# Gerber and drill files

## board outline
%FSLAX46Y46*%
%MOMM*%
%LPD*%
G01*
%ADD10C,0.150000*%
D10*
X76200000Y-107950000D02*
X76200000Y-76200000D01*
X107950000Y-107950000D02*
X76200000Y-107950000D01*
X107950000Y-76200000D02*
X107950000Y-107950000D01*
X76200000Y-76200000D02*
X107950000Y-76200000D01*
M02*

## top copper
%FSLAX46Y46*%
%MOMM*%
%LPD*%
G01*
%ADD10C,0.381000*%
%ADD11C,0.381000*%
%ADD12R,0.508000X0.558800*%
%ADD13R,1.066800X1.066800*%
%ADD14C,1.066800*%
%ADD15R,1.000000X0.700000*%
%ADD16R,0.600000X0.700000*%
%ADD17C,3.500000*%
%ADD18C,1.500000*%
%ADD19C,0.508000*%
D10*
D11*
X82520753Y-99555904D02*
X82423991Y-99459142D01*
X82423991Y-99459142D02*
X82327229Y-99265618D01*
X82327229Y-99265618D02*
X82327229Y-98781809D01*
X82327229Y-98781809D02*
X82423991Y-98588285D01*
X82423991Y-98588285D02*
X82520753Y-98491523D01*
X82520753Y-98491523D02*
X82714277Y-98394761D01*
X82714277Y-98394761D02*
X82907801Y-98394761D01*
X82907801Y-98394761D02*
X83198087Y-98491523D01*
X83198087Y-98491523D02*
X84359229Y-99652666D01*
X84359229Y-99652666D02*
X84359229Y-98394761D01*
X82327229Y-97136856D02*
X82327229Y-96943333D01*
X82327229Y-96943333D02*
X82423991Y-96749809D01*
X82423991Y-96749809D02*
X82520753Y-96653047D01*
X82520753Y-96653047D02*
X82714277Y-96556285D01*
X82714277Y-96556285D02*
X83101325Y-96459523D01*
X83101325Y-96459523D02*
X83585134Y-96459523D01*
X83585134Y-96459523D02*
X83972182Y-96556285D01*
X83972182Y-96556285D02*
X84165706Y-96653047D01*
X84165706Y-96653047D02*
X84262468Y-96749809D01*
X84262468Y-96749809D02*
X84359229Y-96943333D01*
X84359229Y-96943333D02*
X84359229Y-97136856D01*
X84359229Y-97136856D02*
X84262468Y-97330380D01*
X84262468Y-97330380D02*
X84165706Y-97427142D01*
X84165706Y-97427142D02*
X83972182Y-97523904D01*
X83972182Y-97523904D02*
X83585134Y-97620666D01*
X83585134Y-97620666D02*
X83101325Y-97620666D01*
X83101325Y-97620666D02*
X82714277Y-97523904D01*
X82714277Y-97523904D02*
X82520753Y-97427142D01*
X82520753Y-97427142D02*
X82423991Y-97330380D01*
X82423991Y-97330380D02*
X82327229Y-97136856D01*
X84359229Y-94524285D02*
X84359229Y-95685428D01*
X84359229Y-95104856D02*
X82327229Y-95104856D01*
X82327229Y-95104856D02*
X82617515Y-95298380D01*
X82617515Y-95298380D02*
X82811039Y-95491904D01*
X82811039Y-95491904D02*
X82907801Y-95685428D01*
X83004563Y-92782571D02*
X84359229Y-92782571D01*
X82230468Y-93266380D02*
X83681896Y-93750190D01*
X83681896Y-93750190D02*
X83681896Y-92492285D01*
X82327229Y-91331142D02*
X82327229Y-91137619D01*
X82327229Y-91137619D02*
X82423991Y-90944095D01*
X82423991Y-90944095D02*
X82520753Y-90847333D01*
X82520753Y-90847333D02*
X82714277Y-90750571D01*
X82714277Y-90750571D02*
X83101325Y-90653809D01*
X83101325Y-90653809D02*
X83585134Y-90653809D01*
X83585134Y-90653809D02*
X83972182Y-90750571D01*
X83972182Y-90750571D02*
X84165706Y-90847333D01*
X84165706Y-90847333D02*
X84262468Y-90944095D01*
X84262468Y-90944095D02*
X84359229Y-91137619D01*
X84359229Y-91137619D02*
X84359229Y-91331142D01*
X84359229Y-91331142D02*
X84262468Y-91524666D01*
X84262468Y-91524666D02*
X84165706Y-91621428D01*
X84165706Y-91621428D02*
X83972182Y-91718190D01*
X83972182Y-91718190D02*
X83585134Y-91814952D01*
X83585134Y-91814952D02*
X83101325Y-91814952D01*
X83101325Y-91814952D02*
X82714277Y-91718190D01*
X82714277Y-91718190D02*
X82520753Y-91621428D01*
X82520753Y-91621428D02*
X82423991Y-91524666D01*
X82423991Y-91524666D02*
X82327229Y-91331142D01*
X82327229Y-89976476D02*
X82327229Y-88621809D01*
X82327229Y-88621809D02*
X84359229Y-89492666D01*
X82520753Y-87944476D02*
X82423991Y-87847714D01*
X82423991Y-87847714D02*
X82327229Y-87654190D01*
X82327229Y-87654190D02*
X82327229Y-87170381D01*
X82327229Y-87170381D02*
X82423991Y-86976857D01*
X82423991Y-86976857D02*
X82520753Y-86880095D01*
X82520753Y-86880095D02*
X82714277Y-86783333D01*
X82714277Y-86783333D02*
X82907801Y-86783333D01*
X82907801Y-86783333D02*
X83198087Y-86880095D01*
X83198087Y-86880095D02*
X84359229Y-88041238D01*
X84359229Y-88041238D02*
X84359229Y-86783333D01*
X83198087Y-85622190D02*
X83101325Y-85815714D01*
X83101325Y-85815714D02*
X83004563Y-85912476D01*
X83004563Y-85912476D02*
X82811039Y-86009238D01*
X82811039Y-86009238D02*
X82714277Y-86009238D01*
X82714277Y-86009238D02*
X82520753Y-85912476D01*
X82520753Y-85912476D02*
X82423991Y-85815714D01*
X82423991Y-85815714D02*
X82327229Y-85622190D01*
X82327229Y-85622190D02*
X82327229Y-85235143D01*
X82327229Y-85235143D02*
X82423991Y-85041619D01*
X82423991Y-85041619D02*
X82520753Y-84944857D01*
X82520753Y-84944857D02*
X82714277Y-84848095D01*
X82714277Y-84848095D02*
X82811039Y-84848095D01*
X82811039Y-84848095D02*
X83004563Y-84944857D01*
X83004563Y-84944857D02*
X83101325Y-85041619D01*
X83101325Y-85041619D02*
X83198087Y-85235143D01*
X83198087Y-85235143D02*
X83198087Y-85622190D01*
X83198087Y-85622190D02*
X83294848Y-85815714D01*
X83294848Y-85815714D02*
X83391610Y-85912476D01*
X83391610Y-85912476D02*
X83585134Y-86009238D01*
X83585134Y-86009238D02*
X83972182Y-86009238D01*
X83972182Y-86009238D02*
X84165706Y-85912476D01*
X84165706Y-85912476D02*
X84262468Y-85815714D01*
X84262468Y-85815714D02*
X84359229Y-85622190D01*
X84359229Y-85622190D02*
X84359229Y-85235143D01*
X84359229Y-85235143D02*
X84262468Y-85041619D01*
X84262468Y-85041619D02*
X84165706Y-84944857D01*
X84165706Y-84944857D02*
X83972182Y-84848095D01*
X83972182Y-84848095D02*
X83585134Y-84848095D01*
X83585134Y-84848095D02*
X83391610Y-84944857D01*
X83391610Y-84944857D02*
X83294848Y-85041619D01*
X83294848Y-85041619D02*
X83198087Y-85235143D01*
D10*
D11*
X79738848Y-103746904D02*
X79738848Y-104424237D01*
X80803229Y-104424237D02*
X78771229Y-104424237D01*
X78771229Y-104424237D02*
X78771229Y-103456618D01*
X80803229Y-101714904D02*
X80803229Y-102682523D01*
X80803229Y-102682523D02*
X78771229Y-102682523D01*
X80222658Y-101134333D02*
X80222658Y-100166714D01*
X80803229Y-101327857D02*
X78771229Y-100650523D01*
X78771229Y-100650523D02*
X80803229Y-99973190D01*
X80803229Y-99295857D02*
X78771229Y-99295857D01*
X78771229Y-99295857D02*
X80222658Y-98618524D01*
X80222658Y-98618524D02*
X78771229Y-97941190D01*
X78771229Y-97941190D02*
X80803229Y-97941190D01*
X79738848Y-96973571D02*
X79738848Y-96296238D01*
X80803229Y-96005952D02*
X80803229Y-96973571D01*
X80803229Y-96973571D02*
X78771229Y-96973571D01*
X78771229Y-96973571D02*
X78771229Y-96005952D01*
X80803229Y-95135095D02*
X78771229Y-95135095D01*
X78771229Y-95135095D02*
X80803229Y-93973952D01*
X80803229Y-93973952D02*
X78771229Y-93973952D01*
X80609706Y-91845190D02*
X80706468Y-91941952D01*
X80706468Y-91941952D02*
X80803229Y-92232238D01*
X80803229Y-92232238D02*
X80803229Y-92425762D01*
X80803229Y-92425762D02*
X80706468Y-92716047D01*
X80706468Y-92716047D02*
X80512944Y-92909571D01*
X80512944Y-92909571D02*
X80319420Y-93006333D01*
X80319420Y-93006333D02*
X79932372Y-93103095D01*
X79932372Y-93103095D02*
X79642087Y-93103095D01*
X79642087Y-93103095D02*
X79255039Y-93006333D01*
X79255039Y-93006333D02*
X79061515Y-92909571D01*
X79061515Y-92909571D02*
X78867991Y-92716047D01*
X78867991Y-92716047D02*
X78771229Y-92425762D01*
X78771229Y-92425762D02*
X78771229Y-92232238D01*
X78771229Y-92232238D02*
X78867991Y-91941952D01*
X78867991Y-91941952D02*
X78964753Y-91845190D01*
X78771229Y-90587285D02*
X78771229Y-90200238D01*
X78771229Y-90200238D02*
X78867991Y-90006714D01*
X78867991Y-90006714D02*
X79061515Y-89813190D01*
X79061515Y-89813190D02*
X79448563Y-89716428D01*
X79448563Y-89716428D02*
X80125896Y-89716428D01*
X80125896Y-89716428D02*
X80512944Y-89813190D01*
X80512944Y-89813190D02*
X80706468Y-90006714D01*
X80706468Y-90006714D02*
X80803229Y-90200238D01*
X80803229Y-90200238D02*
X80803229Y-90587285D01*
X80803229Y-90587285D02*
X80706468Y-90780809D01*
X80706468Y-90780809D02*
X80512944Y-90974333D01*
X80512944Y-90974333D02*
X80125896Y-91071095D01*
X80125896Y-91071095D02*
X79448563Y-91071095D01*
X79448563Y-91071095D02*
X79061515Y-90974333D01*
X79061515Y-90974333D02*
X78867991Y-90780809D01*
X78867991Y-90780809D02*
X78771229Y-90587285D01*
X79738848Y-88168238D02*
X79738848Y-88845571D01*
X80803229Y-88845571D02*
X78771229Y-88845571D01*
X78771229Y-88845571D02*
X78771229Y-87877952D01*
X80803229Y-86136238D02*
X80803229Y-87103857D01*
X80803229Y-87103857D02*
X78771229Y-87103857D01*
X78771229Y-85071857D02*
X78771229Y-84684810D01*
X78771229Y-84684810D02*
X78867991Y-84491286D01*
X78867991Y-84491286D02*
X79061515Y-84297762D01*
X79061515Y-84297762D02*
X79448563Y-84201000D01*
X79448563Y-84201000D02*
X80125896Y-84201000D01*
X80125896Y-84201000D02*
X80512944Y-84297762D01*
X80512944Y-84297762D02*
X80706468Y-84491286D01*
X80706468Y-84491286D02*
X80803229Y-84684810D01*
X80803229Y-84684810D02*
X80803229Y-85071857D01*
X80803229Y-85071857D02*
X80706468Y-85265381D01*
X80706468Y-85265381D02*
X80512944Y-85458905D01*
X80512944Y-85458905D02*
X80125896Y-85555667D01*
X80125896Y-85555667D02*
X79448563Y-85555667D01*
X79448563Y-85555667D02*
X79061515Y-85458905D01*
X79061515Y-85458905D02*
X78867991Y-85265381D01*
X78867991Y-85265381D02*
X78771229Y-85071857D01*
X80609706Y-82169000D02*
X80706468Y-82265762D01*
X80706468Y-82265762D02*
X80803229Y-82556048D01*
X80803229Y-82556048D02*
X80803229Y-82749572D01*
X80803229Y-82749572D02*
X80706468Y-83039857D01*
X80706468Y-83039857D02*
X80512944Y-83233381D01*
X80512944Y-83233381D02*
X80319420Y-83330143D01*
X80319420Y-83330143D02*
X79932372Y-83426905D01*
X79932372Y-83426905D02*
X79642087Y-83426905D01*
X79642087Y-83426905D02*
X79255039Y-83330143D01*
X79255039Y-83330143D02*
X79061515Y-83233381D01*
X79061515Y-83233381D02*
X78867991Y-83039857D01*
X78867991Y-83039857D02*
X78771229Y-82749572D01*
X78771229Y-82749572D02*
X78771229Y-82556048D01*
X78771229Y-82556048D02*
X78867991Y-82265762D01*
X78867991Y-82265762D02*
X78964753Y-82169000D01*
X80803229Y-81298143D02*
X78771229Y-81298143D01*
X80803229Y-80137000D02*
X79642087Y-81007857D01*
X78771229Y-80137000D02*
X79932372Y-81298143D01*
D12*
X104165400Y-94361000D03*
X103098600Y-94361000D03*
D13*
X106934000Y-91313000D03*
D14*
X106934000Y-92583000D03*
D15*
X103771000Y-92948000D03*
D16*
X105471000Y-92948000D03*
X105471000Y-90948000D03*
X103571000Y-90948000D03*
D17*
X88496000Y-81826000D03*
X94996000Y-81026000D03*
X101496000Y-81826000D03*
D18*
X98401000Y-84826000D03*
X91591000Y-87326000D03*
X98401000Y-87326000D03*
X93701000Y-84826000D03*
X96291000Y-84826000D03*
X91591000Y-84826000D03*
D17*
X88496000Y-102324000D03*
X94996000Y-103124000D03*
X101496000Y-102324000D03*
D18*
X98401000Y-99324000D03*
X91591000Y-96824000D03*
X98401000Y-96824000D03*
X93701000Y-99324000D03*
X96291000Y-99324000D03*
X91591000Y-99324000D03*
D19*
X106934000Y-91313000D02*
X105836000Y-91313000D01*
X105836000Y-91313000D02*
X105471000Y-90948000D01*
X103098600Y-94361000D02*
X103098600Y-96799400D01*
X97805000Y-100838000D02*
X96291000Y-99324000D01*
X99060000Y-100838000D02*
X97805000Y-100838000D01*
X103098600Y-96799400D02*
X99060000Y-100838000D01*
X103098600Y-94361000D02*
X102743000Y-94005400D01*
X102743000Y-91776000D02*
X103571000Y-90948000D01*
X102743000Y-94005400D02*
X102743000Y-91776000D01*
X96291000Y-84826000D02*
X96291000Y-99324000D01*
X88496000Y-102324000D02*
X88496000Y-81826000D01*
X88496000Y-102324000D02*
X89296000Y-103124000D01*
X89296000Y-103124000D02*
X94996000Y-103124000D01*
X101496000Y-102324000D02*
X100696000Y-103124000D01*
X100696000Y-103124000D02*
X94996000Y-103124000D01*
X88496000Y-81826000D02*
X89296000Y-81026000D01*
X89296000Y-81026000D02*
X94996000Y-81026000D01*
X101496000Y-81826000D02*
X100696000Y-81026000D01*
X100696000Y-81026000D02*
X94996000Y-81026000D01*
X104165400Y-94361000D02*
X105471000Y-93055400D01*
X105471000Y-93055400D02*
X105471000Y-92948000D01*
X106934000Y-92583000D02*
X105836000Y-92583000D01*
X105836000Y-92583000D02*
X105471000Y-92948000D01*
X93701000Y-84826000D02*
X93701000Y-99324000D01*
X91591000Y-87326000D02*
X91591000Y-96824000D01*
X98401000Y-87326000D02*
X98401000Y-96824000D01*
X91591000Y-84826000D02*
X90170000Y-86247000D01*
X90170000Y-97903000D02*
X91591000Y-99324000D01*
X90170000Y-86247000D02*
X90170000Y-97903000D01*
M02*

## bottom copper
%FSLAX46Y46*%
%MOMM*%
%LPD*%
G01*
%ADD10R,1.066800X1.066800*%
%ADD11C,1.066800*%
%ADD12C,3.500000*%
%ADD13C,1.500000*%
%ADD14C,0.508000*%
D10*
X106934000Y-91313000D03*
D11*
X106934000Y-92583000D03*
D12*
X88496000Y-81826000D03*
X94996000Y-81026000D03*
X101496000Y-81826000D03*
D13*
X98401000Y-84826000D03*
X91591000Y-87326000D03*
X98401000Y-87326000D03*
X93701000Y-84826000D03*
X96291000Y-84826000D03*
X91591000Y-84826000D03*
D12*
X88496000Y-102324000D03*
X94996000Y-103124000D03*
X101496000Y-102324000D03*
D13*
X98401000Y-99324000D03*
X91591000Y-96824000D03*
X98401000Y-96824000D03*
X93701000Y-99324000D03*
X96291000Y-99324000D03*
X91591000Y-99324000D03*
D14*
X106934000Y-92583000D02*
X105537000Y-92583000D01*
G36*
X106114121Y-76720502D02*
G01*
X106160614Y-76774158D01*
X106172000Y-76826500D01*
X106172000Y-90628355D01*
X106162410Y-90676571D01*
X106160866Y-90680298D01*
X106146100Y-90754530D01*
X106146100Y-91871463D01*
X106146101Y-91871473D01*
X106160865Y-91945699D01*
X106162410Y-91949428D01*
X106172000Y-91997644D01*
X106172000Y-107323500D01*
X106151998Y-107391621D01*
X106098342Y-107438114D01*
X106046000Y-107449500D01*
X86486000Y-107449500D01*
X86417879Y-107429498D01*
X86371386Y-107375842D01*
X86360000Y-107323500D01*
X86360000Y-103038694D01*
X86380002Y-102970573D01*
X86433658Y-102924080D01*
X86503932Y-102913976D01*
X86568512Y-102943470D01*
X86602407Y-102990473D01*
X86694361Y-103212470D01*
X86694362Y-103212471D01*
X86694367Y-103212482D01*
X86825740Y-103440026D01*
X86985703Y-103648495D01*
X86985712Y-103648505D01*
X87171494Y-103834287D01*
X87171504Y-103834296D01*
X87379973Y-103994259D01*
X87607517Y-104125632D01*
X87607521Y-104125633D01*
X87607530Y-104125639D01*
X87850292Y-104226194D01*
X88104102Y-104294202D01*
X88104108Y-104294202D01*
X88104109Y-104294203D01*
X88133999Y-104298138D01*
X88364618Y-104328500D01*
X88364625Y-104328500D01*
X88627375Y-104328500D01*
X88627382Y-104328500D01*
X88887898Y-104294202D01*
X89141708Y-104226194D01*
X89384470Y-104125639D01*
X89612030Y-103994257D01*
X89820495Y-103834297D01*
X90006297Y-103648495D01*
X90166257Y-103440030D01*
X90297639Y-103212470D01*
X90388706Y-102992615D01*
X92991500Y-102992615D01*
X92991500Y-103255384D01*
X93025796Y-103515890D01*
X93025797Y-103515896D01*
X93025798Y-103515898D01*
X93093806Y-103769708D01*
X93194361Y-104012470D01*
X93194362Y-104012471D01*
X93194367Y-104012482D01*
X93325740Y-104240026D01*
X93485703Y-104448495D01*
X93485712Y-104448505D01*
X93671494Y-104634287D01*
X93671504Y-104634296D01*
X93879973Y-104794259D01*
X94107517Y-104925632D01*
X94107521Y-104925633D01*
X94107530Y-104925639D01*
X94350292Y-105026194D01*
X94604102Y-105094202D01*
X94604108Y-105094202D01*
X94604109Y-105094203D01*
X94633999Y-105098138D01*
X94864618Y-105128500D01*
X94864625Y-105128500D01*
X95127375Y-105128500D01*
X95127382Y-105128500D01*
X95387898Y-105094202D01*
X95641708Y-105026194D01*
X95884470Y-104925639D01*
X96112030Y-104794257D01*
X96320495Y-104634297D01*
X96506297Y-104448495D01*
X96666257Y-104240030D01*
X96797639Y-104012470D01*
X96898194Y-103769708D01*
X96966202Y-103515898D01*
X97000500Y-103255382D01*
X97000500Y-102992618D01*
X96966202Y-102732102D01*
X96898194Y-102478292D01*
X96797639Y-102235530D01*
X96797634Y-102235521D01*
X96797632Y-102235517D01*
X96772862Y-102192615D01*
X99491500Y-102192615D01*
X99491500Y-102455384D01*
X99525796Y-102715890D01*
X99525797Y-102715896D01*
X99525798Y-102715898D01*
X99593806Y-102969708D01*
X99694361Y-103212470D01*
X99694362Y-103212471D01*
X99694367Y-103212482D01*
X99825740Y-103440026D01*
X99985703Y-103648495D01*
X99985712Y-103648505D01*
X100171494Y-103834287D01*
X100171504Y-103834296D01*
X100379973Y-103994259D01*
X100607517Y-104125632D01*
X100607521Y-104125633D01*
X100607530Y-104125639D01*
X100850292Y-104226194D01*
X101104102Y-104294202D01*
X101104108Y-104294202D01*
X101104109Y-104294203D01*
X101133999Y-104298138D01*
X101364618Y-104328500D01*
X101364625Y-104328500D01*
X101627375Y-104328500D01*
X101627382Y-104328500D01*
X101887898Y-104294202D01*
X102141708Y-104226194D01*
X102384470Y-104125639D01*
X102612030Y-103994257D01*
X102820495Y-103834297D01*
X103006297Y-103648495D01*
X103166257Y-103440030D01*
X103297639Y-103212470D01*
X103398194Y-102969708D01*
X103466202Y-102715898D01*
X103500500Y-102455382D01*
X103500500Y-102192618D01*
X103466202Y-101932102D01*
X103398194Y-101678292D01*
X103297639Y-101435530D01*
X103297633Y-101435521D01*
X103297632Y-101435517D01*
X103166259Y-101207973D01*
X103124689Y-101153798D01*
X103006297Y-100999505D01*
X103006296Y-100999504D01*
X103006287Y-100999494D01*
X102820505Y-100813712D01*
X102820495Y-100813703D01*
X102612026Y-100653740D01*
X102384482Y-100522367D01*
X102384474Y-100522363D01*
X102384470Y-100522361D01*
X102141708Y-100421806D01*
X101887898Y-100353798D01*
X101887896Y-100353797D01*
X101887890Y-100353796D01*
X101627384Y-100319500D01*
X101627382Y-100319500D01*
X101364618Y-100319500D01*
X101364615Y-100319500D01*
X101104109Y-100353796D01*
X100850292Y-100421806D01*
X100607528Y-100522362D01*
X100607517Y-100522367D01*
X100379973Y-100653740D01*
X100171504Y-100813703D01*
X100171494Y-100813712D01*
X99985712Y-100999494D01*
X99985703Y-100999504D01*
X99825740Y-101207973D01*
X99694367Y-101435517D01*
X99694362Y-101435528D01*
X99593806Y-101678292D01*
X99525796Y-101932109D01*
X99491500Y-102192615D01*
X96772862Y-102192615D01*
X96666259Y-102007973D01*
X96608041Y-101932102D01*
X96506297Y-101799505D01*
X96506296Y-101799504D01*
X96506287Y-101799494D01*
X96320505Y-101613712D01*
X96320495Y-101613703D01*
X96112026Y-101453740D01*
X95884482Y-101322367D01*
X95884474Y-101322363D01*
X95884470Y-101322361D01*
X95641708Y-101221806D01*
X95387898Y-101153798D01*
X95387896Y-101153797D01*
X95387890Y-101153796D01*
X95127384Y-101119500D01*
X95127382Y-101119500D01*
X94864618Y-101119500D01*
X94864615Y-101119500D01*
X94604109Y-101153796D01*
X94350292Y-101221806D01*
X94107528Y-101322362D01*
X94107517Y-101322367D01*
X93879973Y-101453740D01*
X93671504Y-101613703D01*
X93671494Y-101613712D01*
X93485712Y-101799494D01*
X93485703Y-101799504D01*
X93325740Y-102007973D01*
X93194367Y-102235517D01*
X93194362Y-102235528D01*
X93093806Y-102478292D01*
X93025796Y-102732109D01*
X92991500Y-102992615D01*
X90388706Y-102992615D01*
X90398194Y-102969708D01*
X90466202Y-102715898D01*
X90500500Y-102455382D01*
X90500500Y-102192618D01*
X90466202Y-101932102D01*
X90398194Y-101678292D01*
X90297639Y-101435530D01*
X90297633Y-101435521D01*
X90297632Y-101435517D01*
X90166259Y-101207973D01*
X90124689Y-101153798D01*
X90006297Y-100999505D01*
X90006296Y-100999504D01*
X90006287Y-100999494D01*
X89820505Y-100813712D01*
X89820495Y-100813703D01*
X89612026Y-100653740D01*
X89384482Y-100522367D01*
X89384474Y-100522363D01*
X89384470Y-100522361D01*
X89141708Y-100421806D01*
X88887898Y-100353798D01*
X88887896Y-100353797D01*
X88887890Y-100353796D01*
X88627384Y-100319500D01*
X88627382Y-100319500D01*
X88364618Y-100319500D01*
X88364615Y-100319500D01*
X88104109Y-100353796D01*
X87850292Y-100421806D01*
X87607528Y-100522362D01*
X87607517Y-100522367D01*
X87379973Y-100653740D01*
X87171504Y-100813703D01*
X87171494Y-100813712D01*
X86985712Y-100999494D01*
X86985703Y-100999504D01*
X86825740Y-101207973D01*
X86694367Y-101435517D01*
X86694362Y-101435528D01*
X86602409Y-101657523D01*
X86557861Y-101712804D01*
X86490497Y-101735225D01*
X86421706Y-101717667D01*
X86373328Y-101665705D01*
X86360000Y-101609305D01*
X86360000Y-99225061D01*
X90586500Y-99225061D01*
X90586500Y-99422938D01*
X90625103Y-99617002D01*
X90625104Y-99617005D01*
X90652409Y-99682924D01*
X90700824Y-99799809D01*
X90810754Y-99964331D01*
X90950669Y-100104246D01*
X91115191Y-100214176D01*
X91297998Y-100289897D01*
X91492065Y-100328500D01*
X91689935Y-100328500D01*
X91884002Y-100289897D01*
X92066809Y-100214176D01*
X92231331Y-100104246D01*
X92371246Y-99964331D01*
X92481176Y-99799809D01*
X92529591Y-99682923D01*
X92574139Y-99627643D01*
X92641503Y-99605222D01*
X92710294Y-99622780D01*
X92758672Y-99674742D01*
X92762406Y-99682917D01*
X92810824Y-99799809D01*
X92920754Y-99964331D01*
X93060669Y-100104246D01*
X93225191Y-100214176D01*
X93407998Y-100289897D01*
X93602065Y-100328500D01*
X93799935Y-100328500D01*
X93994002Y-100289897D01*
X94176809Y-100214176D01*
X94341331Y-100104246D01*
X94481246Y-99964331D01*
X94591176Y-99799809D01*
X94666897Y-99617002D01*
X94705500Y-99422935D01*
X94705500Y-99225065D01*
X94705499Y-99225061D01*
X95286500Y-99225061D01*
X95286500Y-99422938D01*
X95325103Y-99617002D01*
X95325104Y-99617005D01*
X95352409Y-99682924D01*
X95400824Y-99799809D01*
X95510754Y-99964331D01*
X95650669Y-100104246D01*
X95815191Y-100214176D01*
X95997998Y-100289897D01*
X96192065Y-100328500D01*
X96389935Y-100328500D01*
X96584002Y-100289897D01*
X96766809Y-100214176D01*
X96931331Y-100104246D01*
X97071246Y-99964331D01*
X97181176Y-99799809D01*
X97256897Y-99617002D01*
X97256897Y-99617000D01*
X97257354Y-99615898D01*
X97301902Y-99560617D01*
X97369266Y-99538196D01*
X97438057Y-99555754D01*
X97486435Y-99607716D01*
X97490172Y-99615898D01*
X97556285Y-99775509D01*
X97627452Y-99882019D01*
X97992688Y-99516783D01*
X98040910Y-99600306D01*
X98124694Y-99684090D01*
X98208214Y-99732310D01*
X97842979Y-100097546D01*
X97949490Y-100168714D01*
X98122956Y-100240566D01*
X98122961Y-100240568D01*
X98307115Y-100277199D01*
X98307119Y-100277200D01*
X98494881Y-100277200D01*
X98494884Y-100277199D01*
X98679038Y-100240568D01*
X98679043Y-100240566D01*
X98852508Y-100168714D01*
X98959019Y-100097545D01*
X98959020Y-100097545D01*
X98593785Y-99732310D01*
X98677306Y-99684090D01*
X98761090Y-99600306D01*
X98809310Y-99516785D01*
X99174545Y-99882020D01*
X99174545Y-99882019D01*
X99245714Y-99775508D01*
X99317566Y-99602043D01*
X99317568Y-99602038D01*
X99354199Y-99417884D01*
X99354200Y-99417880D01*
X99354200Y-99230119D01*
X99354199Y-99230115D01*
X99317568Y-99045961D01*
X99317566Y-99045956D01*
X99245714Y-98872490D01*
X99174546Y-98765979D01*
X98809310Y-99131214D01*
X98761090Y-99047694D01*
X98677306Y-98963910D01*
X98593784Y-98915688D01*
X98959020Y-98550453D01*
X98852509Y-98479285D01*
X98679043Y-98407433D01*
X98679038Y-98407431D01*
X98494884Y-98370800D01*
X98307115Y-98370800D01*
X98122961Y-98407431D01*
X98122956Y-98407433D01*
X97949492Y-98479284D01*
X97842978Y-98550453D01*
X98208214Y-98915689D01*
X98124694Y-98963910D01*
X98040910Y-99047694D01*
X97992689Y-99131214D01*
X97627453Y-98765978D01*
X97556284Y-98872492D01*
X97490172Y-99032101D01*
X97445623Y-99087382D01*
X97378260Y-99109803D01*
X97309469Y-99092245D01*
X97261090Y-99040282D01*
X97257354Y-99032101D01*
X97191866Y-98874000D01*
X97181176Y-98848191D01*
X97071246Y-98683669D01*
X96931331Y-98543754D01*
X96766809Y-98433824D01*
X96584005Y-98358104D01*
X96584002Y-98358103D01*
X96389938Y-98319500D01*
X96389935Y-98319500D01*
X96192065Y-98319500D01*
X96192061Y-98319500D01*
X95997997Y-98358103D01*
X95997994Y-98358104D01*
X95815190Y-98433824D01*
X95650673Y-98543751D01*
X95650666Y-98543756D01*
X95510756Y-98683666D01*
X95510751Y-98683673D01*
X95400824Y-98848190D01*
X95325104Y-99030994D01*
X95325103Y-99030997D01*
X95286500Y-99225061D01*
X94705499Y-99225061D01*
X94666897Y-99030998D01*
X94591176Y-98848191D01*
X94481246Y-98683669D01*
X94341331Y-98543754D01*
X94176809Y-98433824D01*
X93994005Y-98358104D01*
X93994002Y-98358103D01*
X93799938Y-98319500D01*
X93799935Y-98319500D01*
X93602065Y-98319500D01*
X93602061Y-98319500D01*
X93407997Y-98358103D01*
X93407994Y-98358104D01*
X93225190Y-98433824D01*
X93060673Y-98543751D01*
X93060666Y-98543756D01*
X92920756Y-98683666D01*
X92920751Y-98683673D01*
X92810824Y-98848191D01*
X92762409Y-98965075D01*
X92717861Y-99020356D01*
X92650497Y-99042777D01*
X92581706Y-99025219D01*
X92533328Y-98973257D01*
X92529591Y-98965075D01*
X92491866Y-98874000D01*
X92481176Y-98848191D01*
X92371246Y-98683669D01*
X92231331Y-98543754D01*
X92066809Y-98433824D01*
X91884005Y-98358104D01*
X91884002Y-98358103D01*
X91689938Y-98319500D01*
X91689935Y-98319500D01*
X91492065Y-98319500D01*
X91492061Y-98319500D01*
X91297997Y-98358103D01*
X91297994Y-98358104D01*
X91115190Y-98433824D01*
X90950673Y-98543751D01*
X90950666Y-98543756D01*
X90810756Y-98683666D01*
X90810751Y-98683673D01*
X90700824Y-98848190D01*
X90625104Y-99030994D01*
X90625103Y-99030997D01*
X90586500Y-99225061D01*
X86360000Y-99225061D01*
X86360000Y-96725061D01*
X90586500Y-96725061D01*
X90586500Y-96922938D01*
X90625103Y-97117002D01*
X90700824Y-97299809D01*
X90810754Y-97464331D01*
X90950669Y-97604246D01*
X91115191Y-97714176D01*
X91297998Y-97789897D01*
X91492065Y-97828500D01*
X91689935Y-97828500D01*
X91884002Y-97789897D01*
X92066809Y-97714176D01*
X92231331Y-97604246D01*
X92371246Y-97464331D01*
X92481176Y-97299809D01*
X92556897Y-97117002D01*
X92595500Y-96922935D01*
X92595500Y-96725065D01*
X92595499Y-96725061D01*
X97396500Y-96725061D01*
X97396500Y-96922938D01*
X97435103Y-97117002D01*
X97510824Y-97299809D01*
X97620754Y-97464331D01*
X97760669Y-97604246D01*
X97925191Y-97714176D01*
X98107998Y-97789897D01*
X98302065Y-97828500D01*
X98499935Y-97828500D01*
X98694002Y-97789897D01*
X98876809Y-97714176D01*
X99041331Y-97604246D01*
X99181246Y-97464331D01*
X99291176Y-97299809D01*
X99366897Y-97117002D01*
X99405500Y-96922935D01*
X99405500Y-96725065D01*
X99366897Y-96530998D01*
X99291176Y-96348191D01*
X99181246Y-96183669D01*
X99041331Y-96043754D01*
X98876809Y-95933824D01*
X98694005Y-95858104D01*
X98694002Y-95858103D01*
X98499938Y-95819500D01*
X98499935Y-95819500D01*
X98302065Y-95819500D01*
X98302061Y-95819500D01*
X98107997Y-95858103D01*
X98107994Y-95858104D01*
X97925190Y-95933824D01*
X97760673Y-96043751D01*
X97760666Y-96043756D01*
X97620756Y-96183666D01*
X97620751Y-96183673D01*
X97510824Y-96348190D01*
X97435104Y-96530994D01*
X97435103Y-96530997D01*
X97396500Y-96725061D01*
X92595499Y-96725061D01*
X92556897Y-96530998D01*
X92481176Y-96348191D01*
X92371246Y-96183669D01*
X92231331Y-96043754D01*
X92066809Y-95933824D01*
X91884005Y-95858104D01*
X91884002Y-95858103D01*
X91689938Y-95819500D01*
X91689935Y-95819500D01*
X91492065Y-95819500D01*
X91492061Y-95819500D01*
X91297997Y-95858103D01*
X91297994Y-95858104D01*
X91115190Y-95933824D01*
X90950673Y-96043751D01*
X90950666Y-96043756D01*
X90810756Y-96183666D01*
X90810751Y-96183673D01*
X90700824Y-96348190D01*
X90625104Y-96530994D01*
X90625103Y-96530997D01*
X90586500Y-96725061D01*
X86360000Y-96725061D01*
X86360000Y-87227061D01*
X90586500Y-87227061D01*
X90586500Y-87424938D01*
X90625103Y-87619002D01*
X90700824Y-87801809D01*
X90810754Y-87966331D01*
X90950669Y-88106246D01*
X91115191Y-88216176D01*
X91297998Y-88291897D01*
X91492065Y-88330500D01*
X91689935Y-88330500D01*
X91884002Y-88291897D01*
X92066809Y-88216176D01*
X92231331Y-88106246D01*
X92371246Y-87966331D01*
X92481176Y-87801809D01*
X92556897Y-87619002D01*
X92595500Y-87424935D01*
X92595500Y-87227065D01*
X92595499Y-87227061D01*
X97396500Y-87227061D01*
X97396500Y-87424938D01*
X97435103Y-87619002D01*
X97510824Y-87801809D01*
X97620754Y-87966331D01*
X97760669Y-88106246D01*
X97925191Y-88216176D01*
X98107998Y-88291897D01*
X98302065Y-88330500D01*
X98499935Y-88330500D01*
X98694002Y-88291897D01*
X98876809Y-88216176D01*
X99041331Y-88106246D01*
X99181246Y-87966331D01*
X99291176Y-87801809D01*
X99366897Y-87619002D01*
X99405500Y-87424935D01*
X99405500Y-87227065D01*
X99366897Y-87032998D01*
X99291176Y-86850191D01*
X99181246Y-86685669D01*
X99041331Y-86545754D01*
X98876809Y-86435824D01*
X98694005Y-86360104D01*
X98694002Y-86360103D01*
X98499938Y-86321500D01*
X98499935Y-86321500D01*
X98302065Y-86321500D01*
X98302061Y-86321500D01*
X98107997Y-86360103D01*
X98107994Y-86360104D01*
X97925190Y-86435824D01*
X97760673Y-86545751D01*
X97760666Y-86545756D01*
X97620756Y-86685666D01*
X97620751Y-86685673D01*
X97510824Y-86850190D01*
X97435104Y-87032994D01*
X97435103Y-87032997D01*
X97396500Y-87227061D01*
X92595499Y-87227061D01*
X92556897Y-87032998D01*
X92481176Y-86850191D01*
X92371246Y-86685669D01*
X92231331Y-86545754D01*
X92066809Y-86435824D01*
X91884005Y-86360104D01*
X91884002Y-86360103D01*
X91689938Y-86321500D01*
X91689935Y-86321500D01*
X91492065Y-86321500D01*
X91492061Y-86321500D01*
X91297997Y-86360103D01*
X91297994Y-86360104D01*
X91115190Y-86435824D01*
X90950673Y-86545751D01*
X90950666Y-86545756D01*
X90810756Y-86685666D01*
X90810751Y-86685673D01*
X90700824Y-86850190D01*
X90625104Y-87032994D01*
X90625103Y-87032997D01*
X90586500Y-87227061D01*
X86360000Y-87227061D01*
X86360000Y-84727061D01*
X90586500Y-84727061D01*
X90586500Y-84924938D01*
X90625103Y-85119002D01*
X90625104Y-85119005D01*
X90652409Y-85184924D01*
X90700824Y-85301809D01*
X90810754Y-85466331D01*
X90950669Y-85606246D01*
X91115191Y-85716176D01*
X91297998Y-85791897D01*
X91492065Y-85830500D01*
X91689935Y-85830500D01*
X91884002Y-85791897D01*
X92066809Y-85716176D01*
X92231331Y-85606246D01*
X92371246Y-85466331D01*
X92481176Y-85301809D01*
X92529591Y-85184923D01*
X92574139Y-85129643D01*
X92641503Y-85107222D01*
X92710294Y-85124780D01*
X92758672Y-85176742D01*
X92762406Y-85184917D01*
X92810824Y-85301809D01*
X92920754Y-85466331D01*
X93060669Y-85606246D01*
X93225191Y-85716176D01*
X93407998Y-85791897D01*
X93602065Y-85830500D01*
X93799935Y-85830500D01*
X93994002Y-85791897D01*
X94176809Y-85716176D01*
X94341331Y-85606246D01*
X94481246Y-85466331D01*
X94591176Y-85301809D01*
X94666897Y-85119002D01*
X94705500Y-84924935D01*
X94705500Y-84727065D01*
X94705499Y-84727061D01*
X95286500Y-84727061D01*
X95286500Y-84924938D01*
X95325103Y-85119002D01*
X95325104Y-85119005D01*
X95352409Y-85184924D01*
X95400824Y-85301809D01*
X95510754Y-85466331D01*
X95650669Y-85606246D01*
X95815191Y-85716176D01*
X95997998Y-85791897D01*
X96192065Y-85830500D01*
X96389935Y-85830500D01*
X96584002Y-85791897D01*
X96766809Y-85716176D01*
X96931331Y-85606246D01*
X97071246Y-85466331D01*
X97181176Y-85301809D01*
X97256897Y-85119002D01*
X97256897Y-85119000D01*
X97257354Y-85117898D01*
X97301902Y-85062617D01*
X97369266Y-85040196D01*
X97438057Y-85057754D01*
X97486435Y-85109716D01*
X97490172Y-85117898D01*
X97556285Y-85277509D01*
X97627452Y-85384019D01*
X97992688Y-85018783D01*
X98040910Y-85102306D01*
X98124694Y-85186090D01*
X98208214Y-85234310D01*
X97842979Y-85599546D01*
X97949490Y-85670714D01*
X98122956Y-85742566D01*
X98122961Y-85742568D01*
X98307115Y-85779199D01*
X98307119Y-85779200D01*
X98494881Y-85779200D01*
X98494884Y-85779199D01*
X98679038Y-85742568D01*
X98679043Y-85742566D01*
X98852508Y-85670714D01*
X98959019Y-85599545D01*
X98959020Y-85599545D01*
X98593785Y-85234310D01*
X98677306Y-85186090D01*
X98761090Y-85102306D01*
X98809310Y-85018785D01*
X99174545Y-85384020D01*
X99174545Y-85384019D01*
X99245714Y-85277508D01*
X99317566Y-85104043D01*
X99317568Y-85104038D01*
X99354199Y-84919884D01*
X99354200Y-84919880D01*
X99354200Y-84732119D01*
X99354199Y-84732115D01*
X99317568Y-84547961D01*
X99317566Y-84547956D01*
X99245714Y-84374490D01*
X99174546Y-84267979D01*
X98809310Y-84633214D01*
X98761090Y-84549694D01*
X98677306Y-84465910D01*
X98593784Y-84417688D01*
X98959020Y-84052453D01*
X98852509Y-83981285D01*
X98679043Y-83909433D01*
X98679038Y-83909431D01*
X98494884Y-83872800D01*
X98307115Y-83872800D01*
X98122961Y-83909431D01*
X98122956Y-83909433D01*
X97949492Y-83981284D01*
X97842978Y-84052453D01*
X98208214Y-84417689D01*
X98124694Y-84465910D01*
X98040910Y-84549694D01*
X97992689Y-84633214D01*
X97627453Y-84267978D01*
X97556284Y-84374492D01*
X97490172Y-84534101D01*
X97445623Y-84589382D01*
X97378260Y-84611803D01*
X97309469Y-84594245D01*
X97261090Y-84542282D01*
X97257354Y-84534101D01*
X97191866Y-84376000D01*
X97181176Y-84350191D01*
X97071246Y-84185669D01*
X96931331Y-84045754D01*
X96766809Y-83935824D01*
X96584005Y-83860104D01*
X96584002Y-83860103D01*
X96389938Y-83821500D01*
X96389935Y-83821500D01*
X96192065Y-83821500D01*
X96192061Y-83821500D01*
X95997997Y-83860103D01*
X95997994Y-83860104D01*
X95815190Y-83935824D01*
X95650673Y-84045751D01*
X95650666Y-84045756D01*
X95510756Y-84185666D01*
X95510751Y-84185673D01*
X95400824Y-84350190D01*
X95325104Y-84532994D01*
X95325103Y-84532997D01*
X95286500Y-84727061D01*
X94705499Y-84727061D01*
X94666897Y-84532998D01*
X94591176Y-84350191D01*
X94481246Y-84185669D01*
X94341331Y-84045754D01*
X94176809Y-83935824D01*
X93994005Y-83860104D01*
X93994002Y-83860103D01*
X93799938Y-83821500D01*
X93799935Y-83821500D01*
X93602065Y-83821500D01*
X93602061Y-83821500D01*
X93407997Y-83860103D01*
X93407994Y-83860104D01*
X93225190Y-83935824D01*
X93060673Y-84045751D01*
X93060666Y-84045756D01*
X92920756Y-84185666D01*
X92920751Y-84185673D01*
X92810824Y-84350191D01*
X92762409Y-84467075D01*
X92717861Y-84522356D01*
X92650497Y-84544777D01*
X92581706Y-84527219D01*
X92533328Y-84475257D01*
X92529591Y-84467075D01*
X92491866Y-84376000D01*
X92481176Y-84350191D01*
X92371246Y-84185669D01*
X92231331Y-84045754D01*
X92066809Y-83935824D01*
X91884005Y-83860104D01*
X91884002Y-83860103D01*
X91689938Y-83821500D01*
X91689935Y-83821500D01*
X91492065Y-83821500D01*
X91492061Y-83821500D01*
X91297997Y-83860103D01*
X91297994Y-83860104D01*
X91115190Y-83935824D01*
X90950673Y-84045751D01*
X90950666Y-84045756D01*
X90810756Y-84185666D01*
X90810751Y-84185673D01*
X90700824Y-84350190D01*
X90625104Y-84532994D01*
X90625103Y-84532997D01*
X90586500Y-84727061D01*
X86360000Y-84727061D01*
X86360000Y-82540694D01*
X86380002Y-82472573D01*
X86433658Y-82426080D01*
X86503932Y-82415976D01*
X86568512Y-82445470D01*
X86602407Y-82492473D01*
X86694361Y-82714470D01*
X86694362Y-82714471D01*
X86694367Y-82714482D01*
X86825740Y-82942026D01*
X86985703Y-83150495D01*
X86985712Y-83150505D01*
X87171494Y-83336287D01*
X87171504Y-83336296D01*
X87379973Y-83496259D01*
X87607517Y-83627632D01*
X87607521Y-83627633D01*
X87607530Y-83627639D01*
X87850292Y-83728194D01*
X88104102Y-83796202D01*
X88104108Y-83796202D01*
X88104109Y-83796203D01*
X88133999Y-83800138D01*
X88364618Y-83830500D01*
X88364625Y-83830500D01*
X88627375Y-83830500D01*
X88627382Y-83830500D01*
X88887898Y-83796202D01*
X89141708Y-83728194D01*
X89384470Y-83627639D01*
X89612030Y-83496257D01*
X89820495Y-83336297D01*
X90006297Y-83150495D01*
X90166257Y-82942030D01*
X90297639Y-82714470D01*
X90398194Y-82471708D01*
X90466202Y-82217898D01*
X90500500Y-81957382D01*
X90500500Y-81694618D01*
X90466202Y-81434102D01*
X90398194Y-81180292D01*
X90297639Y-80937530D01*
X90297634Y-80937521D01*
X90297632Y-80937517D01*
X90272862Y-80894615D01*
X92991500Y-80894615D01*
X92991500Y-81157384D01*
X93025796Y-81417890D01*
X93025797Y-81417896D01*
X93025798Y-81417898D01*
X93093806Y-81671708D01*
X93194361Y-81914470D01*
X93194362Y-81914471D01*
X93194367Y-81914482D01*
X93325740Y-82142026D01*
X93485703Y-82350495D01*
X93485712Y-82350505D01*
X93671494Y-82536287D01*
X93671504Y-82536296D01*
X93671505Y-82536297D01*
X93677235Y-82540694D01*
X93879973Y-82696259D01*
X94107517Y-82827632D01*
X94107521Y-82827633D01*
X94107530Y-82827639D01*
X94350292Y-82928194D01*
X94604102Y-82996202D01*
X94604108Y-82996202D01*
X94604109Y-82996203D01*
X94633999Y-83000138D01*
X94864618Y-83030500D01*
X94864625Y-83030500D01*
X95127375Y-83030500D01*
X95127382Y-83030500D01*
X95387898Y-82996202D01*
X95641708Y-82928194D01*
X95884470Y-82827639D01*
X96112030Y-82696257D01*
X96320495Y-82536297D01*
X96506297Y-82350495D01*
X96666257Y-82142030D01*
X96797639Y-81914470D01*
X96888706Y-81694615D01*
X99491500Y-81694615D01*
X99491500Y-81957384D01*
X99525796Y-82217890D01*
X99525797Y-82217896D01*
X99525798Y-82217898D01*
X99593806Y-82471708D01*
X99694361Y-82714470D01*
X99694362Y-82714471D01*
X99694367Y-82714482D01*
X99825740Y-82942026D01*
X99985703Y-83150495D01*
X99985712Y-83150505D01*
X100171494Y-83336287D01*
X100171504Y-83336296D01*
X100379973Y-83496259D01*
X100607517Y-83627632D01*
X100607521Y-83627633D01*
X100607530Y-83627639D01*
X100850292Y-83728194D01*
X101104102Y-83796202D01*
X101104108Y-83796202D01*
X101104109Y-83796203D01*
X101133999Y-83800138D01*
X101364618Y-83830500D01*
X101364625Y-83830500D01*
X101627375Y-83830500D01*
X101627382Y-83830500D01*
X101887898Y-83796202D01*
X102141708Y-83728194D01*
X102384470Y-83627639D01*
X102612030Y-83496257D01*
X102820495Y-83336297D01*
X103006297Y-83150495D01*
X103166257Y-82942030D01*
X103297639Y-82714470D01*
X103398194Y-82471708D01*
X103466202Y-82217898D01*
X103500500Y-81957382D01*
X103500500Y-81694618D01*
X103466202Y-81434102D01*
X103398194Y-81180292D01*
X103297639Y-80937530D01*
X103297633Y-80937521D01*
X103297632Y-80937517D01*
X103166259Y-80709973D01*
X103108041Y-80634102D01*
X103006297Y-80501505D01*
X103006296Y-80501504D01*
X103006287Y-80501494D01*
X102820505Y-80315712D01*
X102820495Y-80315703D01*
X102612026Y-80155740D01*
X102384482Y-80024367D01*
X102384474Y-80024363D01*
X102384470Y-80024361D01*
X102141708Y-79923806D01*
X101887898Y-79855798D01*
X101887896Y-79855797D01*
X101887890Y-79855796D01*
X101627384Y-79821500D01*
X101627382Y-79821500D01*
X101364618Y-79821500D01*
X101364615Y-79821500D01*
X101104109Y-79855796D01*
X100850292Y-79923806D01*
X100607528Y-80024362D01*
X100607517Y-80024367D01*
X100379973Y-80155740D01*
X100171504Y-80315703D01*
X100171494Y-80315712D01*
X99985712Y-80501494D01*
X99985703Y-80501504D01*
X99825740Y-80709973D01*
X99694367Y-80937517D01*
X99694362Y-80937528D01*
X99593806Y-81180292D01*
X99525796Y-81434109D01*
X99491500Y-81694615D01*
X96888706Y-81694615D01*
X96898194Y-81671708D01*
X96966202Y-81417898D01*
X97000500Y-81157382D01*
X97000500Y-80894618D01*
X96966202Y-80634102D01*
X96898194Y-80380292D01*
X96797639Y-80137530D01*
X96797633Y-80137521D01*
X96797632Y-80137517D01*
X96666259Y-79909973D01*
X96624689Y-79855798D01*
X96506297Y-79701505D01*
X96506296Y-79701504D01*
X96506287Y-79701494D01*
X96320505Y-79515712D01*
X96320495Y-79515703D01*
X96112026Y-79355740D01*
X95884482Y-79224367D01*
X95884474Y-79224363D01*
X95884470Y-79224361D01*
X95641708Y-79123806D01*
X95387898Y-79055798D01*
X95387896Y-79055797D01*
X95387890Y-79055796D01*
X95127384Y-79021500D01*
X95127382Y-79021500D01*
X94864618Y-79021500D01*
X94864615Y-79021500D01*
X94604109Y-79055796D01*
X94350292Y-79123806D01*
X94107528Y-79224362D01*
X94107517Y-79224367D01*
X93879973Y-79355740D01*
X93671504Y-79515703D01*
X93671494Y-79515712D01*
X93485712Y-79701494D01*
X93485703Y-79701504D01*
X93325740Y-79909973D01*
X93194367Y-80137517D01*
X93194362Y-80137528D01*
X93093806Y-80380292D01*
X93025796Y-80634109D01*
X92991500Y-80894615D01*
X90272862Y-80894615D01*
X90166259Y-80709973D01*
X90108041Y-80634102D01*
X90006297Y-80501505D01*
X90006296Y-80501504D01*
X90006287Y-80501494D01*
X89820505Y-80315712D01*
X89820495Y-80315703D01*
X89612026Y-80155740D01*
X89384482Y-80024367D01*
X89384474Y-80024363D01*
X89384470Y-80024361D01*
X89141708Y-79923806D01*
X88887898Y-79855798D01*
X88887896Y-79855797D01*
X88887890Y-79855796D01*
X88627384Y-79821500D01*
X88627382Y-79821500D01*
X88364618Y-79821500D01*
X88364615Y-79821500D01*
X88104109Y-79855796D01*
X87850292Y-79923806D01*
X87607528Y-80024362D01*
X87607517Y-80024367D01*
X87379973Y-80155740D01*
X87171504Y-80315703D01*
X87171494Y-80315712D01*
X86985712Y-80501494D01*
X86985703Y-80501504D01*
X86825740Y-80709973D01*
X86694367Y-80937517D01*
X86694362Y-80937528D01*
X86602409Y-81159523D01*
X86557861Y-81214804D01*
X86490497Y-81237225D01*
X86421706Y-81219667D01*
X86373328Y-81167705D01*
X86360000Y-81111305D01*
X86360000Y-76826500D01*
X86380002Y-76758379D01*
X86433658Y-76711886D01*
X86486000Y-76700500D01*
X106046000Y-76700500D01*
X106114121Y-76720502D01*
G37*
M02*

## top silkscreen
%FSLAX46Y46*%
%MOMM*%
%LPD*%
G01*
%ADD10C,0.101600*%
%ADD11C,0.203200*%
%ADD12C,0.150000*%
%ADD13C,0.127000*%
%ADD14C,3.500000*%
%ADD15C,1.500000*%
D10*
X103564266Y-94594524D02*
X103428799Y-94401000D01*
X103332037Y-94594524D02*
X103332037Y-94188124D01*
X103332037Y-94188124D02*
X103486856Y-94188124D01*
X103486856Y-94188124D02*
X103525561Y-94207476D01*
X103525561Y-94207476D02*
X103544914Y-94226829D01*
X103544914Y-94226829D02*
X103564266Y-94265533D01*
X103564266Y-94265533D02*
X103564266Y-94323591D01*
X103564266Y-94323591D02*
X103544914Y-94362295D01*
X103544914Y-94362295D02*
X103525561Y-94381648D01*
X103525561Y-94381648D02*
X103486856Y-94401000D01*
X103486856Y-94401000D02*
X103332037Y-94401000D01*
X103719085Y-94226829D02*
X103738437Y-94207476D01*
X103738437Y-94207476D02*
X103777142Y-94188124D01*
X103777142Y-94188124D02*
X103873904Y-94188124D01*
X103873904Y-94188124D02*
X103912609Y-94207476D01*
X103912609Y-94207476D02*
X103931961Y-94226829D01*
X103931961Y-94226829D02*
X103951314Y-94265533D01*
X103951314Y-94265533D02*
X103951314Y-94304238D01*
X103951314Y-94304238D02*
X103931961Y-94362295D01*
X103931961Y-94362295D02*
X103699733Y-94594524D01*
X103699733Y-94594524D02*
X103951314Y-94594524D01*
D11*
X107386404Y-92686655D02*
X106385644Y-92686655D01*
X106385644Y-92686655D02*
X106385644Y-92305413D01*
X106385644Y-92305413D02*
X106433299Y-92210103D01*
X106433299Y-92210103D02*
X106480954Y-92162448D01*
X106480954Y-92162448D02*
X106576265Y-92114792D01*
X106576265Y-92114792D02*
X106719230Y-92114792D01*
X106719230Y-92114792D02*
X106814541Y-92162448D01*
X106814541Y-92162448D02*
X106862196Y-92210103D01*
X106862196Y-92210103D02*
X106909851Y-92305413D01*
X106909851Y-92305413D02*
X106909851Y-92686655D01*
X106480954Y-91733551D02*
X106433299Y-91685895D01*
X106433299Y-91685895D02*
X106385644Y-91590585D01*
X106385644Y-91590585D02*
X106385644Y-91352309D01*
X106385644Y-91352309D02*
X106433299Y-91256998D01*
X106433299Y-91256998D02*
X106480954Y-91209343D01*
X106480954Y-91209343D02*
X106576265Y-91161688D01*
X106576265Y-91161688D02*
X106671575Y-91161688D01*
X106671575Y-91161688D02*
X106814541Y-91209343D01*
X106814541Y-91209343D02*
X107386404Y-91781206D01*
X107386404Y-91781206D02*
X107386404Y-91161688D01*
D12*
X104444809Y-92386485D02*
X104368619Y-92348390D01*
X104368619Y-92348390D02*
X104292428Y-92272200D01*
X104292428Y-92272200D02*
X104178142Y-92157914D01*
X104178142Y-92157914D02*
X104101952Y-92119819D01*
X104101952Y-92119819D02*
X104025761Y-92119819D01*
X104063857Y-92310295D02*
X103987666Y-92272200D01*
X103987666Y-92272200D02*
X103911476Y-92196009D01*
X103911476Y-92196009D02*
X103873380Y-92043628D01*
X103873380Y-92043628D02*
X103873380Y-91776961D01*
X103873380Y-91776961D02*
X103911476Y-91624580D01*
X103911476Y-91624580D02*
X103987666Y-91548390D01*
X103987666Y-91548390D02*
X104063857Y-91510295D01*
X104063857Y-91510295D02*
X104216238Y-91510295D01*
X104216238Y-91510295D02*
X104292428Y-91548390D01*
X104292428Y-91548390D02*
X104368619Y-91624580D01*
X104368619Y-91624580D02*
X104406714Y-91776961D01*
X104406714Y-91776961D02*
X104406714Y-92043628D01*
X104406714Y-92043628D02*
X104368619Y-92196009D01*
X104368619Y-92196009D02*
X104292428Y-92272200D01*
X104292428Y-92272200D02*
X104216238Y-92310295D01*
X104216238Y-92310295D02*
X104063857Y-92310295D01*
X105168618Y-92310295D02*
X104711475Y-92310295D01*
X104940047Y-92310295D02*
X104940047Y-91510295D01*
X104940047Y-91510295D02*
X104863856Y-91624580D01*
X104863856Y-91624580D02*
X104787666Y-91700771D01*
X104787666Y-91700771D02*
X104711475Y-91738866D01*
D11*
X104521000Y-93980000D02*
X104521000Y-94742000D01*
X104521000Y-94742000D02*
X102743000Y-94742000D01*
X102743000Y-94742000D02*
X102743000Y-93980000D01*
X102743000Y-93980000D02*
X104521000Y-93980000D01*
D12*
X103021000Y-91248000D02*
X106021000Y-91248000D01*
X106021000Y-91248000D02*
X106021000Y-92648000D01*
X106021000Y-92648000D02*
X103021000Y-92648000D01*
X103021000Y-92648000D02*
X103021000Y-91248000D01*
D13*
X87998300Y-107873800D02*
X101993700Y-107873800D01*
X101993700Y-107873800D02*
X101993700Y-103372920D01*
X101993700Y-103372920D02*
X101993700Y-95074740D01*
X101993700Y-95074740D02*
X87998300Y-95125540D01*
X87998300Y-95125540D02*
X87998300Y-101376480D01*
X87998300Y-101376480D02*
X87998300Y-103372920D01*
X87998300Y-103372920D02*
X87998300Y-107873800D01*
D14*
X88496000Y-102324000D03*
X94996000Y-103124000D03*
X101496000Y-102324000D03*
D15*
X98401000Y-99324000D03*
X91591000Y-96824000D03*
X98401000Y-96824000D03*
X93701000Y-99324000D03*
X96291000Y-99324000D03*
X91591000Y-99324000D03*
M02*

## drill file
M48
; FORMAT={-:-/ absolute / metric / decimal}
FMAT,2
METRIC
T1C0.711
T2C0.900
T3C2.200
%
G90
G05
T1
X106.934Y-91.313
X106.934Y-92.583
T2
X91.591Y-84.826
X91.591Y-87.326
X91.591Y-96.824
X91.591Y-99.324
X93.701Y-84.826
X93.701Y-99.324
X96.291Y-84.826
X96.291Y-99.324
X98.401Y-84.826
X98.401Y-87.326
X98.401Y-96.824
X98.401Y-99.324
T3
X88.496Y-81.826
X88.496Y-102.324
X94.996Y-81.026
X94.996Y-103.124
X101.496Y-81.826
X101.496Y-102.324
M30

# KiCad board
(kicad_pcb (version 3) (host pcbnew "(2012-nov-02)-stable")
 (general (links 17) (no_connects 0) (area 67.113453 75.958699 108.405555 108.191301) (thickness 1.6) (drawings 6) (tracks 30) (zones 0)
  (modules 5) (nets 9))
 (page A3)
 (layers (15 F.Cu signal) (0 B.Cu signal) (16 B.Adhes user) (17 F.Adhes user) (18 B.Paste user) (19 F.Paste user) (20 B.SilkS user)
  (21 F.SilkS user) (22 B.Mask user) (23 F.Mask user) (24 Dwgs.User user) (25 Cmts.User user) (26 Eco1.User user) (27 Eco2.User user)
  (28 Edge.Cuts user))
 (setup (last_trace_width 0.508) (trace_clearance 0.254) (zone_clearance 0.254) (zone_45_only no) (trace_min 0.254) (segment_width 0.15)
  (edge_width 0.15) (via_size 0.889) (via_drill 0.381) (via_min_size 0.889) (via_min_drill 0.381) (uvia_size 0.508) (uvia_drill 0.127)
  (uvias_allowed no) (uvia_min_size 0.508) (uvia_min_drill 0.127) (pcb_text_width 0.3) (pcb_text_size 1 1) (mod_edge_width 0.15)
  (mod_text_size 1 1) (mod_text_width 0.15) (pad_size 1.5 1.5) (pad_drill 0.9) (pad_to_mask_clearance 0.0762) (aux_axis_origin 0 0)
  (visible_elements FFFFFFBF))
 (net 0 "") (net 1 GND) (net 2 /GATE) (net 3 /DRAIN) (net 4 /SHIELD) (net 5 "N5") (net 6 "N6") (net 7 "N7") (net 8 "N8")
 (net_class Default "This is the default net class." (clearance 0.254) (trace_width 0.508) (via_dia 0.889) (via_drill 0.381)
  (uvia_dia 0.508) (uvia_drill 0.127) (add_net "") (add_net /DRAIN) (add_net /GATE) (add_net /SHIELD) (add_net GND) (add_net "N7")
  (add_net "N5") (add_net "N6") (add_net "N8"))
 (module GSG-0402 (layer F.Cu) (at 103.632 94.361) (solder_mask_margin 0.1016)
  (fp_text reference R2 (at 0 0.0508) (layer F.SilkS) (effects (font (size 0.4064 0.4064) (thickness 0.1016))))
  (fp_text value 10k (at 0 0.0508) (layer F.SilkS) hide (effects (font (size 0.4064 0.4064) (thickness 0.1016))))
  (fp_line (start 0.889 -0.381) (end 0.889 0.381) (layer F.SilkS) (width 0.2032))
  (fp_line (start 0.889 0.381) (end -0.889 0.381) (layer F.SilkS) (width 0.2032))
  (fp_line (start -0.889 0.381) (end -0.889 -0.381) (layer F.SilkS) (width 0.2032))
  (fp_line (start -0.889 -0.381) (end 0.889 -0.381) (layer F.SilkS) (width 0.2032))
  (pad 2 smd rect (at 0.5334 0) (size 0.508 0.5588) (layers F.Cu F.Paste F.Mask) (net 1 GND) (solder_mask_margin 0.1016))
  (pad 1 smd rect (at -0.5334 0) (size 0.508 0.5588) (layers F.Cu F.Paste F.Mask) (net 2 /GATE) (die_length -2147.483648)
   (solder_mask_margin 0.1016)))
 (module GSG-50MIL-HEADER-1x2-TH (layer F.Cu) (at 106.934 91.948 270)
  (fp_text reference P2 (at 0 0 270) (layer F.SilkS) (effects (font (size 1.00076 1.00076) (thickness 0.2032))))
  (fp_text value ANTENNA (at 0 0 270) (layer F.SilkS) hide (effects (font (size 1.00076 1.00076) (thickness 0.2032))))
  (pad 1 thru_hole rect (at -0.635 0 270) (size 1.0668 1.0668) (drill 0.7112) (layers *.Cu *.Mask) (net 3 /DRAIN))
  (pad 2 thru_hole circle (at 0.635 0 270) (size 1.0668 1.0668) (drill 0.7112) (layers *.Cu *.Mask) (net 1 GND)))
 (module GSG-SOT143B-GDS (layer F.Cu) (at 104.521 91.948)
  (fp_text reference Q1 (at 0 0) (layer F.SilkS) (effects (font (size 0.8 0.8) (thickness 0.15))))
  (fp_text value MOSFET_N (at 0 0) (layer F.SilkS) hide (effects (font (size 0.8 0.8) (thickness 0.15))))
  (fp_line (start -1.5 -0.7) (end 1.5 -0.7) (layer F.SilkS) (width 0.15))
  (fp_line (start 1.5 -0.7) (end 1.5 0.7) (layer F.SilkS) (width 0.15))
  (fp_line (start 1.5 0.7) (end -1.5 0.7) (layer F.SilkS) (width 0.15))
  (fp_line (start -1.5 0.7) (end -1.5 -0.7) (layer F.SilkS) (width 0.15))
  (pad B smd rect (at -0.75 1) (size 1 0.7) (layers F.Cu F.Paste F.Mask))
  (pad S smd rect (at 0.95 1) (size 0.6 0.7) (layers F.Cu F.Paste F.Mask) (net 1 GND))
  (pad D smd rect (at 0.95 -1) (size 0.6 0.7) (layers F.Cu F.Paste F.Mask) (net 3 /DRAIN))
  (pad G smd rect (at -0.95 -1) (size 0.6 0.7) (layers F.Cu F.Paste F.Mask) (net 2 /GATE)))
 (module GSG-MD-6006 (layer B.Cu) (at 94.996 81.026 180)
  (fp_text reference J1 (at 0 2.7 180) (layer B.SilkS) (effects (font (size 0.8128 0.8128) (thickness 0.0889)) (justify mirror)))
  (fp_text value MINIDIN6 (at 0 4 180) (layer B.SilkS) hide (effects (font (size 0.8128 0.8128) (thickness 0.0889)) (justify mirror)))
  (pad 0 thru_hole circle (at 6.5 -0.8 180) (size 3.5 3.5) (drill 2.2) (layers *.Cu *.Mask B.SilkS) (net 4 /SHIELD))
  (pad 0 thru_hole circle (at 0 0 180) (size 3.5 3.5) (drill 2.2) (layers *.Cu *.Mask B.SilkS) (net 4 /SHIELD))
  (pad 0 thru_hole circle (at -6.5 -0.8 180) (size 3.5 3.5) (drill 2.2) (layers *.Cu *.Mask B.SilkS) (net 4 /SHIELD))
  (pad 3 thru_hole circle (at -3.405 -3.8 180) (size 1.5 1.5) (drill 0.9) (layers *.Cu *.Mask B.SilkS) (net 1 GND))
  (pad 6 thru_hole circle (at 3.405 -6.3 180) (size 1.5 1.5) (drill 0.9) (layers *.Cu *.Mask B.SilkS) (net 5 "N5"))
  (pad 5 thru_hole circle (at -3.405 -6.3 180) (size 1.5 1.5) (drill 0.9) (layers *.Cu *.Mask B.SilkS) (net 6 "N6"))
  (pad 2 thru_hole circle (at 1.295 -3.8 180) (size 1.5 1.5) (drill 0.9) (layers *.Cu *.Mask B.SilkS) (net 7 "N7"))
  (pad 1 thru_hole circle (at -1.295 -3.8 180) (size 1.5 1.5) (drill 0.9) (layers *.Cu *.Mask B.SilkS) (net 2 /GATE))
  (pad 4 thru_hole circle (at 3.405 -3.8 180) (size 1.5 1.5) (drill 0.9) (layers *.Cu *.Mask B.SilkS) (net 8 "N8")))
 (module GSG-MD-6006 (layer F.Cu) (at 94.996 103.124 180)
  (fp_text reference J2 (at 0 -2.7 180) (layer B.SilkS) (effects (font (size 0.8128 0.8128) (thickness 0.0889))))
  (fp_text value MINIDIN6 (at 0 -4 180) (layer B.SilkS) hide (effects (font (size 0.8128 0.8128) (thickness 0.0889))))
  (fp_line (start 6.9977 -4.7498) (end -6.9977 -4.7498) (layer F.SilkS) (width 0.127))
  (fp_line (start -6.9977 -4.7498) (end -6.9977 -0.24892) (layer F.SilkS) (width 0.127))
  (fp_line (start -6.9977 -0.24892) (end -6.9977 8.04926) (layer F.SilkS) (width 0.127))
  (fp_line (start -6.9977 8.04926) (end 6.9977 7.99846) (layer F.SilkS) (width 0.127))
  (fp_line (start 6.9977 7.99846) (end 6.9977 1.74752) (layer F.SilkS) (width 0.127))
  (fp_line (start 6.9977 1.74752) (end 6.9977 -0.24892) (layer F.SilkS) (width 0.127))
  (fp_line (start 6.9977 -0.24892) (end 6.9977 -4.7498) (layer F.SilkS) (width 0.127))
  (pad 0 thru_hole circle (at 6.5 0.8 180) (size 3.5 3.5) (drill 2.2) (layers *.Cu *.Mask F.SilkS) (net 4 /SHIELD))
  (pad 0 thru_hole circle (at 0 0 180) (size 3.5 3.5) (drill 2.2) (layers *.Cu *.Mask F.SilkS) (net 4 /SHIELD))
  (pad 0 thru_hole circle (at -6.5 0.8 180) (size 3.5 3.5) (drill 2.2) (layers *.Cu *.Mask F.SilkS) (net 4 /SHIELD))
  (pad 3 thru_hole circle (at -3.405 3.8 180) (size 1.5 1.5) (drill 0.9) (layers *.Cu *.Mask F.SilkS) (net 1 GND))
  (pad 6 thru_hole circle (at 3.405 6.3 180) (size 1.5 1.5) (drill 0.9) (layers *.Cu *.Mask F.SilkS) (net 5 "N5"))
  (pad 5 thru_hole circle (at -3.405 6.3 180) (size 1.5 1.5) (drill 0.9) (layers *.Cu *.Mask F.SilkS) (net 6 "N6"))
  (pad 2 thru_hole circle (at 1.295 3.8 180) (size 1.5 1.5) (drill 0.9) (layers *.Cu *.Mask F.SilkS) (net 7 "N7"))
  (pad 1 thru_hole circle (at -1.295 3.8 180) (size 1.5 1.5) (drill 0.9) (layers *.Cu *.Mask F.SilkS) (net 2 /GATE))
  (pad 4 thru_hole circle (at 3.405 3.8 180) (size 1.5 1.5) (drill 0.9) (layers *.Cu *.Mask F.SilkS) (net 8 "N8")))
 (gr_line (start 76.2 107.95) (end 76.2 76.2) (angle 90) (layer Edge.Cuts) (width 0.15))
 (gr_line (start 107.95 107.95) (end 76.2 107.95) (angle 90) (layer Edge.Cuts) (width 0.15))
 (gr_line (start 107.95 76.2) (end 107.95 107.95) (angle 90) (layer Edge.Cuts) (width 0.15))
 (gr_line (start 76.2 76.2) (end 107.95 76.2) (angle 90) (layer Edge.Cuts) (width 0.15))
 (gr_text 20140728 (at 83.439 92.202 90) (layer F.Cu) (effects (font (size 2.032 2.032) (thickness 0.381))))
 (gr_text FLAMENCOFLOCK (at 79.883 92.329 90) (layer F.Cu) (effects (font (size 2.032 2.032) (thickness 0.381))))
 (segment (start 106.934 91.313) (end 105.836 91.313) (width 0.508) (layer F.Cu) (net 3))
 (segment (start 105.836 91.313) (end 105.471 90.948) (width 0.508) (layer F.Cu) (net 3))
 (segment (start 103.0986 94.361) (end 103.0986 96.7994) (width 0.508) (layer F.Cu) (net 2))
 (segment (start 97.805 100.838) (end 96.291 99.324) (width 0.508) (layer F.Cu) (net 2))
 (segment (start 99.06 100.838) (end 97.805 100.838) (width 0.508) (layer F.Cu) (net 2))
 (segment (start 103.0986 96.7994) (end 99.06 100.838) (width 0.508) (layer F.Cu) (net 2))
 (segment (start 103.0986 94.361) (end 102.743 94.0054) (width 0.508) (layer F.Cu) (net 2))
 (segment (start 102.743 91.776) (end 103.571 90.948) (width 0.508) (layer F.Cu) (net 2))
 (segment (start 102.743 94.0054) (end 102.743 91.776) (width 0.508) (layer F.Cu) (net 2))
 (segment (start 96.291 84.826) (end 96.291 99.324) (width 0.508) (layer F.Cu) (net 2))
 (segment (start 88.496 102.324) (end 88.496 81.826) (width 0.508) (layer F.Cu) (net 4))
 (segment (start 88.496 102.324) (end 89.296 103.124) (width 0.508) (layer F.Cu) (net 4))
 (segment (start 89.296 103.124) (end 94.996 103.124) (width 0.508) (layer F.Cu) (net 4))
 (segment (start 101.496 102.324) (end 100.696 103.124) (width 0.508) (layer F.Cu) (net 4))
 (segment (start 100.696 103.124) (end 94.996 103.124) (width 0.508) (layer F.Cu) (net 4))
 (segment (start 88.496 81.826) (end 89.296 81.026) (width 0.508) (layer F.Cu) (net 4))
 (segment (start 89.296 81.026) (end 94.996 81.026) (width 0.508) (layer F.Cu) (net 4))
 (segment (start 101.496 81.826) (end 100.696 81.026) (width 0.508) (layer F.Cu) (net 4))
 (segment (start 100.696 81.026) (end 94.996 81.026) (width 0.508) (layer F.Cu) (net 4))
 (segment (start 104.1654 94.361) (end 105.471 93.0554) (width 0.508) (layer F.Cu) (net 1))
 (segment (start 105.471 93.0554) (end 105.471 92.948) (width 0.508) (layer F.Cu) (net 1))
 (segment (start 106.934 92.583) (end 105.836 92.583) (width 0.508) (layer F.Cu) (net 1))
 (segment (start 105.836 92.583) (end 105.471 92.948) (width 0.508) (layer F.Cu) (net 1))
 (segment (start 106.934 92.583) (end 105.537 92.583) (width 0.508) (layer B.Cu) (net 1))
 (segment (start 93.701 84.826) (end 93.701 99.324) (width 0.508) (layer F.Cu) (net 7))
 (segment (start 91.591 87.326) (end 91.591 96.824) (width 0.508) (layer F.Cu) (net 5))
 (segment (start 98.401 87.326) (end 98.401 96.824) (width 0.508) (layer F.Cu) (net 6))
 (segment (start 91.591 84.826) (end 90.17 86.247) (width 0.508) (layer F.Cu) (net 8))
 (segment (start 90.17 97.903) (end 91.591 99.324) (width 0.508) (layer F.Cu) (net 8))
 (segment (start 90.17 86.247) (end 90.17 97.903) (width 0.508) (layer F.Cu) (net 8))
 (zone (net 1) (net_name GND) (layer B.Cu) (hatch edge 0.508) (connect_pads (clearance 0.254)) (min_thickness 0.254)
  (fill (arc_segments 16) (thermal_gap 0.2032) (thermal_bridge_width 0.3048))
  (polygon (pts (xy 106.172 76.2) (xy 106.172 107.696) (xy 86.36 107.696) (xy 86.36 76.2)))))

